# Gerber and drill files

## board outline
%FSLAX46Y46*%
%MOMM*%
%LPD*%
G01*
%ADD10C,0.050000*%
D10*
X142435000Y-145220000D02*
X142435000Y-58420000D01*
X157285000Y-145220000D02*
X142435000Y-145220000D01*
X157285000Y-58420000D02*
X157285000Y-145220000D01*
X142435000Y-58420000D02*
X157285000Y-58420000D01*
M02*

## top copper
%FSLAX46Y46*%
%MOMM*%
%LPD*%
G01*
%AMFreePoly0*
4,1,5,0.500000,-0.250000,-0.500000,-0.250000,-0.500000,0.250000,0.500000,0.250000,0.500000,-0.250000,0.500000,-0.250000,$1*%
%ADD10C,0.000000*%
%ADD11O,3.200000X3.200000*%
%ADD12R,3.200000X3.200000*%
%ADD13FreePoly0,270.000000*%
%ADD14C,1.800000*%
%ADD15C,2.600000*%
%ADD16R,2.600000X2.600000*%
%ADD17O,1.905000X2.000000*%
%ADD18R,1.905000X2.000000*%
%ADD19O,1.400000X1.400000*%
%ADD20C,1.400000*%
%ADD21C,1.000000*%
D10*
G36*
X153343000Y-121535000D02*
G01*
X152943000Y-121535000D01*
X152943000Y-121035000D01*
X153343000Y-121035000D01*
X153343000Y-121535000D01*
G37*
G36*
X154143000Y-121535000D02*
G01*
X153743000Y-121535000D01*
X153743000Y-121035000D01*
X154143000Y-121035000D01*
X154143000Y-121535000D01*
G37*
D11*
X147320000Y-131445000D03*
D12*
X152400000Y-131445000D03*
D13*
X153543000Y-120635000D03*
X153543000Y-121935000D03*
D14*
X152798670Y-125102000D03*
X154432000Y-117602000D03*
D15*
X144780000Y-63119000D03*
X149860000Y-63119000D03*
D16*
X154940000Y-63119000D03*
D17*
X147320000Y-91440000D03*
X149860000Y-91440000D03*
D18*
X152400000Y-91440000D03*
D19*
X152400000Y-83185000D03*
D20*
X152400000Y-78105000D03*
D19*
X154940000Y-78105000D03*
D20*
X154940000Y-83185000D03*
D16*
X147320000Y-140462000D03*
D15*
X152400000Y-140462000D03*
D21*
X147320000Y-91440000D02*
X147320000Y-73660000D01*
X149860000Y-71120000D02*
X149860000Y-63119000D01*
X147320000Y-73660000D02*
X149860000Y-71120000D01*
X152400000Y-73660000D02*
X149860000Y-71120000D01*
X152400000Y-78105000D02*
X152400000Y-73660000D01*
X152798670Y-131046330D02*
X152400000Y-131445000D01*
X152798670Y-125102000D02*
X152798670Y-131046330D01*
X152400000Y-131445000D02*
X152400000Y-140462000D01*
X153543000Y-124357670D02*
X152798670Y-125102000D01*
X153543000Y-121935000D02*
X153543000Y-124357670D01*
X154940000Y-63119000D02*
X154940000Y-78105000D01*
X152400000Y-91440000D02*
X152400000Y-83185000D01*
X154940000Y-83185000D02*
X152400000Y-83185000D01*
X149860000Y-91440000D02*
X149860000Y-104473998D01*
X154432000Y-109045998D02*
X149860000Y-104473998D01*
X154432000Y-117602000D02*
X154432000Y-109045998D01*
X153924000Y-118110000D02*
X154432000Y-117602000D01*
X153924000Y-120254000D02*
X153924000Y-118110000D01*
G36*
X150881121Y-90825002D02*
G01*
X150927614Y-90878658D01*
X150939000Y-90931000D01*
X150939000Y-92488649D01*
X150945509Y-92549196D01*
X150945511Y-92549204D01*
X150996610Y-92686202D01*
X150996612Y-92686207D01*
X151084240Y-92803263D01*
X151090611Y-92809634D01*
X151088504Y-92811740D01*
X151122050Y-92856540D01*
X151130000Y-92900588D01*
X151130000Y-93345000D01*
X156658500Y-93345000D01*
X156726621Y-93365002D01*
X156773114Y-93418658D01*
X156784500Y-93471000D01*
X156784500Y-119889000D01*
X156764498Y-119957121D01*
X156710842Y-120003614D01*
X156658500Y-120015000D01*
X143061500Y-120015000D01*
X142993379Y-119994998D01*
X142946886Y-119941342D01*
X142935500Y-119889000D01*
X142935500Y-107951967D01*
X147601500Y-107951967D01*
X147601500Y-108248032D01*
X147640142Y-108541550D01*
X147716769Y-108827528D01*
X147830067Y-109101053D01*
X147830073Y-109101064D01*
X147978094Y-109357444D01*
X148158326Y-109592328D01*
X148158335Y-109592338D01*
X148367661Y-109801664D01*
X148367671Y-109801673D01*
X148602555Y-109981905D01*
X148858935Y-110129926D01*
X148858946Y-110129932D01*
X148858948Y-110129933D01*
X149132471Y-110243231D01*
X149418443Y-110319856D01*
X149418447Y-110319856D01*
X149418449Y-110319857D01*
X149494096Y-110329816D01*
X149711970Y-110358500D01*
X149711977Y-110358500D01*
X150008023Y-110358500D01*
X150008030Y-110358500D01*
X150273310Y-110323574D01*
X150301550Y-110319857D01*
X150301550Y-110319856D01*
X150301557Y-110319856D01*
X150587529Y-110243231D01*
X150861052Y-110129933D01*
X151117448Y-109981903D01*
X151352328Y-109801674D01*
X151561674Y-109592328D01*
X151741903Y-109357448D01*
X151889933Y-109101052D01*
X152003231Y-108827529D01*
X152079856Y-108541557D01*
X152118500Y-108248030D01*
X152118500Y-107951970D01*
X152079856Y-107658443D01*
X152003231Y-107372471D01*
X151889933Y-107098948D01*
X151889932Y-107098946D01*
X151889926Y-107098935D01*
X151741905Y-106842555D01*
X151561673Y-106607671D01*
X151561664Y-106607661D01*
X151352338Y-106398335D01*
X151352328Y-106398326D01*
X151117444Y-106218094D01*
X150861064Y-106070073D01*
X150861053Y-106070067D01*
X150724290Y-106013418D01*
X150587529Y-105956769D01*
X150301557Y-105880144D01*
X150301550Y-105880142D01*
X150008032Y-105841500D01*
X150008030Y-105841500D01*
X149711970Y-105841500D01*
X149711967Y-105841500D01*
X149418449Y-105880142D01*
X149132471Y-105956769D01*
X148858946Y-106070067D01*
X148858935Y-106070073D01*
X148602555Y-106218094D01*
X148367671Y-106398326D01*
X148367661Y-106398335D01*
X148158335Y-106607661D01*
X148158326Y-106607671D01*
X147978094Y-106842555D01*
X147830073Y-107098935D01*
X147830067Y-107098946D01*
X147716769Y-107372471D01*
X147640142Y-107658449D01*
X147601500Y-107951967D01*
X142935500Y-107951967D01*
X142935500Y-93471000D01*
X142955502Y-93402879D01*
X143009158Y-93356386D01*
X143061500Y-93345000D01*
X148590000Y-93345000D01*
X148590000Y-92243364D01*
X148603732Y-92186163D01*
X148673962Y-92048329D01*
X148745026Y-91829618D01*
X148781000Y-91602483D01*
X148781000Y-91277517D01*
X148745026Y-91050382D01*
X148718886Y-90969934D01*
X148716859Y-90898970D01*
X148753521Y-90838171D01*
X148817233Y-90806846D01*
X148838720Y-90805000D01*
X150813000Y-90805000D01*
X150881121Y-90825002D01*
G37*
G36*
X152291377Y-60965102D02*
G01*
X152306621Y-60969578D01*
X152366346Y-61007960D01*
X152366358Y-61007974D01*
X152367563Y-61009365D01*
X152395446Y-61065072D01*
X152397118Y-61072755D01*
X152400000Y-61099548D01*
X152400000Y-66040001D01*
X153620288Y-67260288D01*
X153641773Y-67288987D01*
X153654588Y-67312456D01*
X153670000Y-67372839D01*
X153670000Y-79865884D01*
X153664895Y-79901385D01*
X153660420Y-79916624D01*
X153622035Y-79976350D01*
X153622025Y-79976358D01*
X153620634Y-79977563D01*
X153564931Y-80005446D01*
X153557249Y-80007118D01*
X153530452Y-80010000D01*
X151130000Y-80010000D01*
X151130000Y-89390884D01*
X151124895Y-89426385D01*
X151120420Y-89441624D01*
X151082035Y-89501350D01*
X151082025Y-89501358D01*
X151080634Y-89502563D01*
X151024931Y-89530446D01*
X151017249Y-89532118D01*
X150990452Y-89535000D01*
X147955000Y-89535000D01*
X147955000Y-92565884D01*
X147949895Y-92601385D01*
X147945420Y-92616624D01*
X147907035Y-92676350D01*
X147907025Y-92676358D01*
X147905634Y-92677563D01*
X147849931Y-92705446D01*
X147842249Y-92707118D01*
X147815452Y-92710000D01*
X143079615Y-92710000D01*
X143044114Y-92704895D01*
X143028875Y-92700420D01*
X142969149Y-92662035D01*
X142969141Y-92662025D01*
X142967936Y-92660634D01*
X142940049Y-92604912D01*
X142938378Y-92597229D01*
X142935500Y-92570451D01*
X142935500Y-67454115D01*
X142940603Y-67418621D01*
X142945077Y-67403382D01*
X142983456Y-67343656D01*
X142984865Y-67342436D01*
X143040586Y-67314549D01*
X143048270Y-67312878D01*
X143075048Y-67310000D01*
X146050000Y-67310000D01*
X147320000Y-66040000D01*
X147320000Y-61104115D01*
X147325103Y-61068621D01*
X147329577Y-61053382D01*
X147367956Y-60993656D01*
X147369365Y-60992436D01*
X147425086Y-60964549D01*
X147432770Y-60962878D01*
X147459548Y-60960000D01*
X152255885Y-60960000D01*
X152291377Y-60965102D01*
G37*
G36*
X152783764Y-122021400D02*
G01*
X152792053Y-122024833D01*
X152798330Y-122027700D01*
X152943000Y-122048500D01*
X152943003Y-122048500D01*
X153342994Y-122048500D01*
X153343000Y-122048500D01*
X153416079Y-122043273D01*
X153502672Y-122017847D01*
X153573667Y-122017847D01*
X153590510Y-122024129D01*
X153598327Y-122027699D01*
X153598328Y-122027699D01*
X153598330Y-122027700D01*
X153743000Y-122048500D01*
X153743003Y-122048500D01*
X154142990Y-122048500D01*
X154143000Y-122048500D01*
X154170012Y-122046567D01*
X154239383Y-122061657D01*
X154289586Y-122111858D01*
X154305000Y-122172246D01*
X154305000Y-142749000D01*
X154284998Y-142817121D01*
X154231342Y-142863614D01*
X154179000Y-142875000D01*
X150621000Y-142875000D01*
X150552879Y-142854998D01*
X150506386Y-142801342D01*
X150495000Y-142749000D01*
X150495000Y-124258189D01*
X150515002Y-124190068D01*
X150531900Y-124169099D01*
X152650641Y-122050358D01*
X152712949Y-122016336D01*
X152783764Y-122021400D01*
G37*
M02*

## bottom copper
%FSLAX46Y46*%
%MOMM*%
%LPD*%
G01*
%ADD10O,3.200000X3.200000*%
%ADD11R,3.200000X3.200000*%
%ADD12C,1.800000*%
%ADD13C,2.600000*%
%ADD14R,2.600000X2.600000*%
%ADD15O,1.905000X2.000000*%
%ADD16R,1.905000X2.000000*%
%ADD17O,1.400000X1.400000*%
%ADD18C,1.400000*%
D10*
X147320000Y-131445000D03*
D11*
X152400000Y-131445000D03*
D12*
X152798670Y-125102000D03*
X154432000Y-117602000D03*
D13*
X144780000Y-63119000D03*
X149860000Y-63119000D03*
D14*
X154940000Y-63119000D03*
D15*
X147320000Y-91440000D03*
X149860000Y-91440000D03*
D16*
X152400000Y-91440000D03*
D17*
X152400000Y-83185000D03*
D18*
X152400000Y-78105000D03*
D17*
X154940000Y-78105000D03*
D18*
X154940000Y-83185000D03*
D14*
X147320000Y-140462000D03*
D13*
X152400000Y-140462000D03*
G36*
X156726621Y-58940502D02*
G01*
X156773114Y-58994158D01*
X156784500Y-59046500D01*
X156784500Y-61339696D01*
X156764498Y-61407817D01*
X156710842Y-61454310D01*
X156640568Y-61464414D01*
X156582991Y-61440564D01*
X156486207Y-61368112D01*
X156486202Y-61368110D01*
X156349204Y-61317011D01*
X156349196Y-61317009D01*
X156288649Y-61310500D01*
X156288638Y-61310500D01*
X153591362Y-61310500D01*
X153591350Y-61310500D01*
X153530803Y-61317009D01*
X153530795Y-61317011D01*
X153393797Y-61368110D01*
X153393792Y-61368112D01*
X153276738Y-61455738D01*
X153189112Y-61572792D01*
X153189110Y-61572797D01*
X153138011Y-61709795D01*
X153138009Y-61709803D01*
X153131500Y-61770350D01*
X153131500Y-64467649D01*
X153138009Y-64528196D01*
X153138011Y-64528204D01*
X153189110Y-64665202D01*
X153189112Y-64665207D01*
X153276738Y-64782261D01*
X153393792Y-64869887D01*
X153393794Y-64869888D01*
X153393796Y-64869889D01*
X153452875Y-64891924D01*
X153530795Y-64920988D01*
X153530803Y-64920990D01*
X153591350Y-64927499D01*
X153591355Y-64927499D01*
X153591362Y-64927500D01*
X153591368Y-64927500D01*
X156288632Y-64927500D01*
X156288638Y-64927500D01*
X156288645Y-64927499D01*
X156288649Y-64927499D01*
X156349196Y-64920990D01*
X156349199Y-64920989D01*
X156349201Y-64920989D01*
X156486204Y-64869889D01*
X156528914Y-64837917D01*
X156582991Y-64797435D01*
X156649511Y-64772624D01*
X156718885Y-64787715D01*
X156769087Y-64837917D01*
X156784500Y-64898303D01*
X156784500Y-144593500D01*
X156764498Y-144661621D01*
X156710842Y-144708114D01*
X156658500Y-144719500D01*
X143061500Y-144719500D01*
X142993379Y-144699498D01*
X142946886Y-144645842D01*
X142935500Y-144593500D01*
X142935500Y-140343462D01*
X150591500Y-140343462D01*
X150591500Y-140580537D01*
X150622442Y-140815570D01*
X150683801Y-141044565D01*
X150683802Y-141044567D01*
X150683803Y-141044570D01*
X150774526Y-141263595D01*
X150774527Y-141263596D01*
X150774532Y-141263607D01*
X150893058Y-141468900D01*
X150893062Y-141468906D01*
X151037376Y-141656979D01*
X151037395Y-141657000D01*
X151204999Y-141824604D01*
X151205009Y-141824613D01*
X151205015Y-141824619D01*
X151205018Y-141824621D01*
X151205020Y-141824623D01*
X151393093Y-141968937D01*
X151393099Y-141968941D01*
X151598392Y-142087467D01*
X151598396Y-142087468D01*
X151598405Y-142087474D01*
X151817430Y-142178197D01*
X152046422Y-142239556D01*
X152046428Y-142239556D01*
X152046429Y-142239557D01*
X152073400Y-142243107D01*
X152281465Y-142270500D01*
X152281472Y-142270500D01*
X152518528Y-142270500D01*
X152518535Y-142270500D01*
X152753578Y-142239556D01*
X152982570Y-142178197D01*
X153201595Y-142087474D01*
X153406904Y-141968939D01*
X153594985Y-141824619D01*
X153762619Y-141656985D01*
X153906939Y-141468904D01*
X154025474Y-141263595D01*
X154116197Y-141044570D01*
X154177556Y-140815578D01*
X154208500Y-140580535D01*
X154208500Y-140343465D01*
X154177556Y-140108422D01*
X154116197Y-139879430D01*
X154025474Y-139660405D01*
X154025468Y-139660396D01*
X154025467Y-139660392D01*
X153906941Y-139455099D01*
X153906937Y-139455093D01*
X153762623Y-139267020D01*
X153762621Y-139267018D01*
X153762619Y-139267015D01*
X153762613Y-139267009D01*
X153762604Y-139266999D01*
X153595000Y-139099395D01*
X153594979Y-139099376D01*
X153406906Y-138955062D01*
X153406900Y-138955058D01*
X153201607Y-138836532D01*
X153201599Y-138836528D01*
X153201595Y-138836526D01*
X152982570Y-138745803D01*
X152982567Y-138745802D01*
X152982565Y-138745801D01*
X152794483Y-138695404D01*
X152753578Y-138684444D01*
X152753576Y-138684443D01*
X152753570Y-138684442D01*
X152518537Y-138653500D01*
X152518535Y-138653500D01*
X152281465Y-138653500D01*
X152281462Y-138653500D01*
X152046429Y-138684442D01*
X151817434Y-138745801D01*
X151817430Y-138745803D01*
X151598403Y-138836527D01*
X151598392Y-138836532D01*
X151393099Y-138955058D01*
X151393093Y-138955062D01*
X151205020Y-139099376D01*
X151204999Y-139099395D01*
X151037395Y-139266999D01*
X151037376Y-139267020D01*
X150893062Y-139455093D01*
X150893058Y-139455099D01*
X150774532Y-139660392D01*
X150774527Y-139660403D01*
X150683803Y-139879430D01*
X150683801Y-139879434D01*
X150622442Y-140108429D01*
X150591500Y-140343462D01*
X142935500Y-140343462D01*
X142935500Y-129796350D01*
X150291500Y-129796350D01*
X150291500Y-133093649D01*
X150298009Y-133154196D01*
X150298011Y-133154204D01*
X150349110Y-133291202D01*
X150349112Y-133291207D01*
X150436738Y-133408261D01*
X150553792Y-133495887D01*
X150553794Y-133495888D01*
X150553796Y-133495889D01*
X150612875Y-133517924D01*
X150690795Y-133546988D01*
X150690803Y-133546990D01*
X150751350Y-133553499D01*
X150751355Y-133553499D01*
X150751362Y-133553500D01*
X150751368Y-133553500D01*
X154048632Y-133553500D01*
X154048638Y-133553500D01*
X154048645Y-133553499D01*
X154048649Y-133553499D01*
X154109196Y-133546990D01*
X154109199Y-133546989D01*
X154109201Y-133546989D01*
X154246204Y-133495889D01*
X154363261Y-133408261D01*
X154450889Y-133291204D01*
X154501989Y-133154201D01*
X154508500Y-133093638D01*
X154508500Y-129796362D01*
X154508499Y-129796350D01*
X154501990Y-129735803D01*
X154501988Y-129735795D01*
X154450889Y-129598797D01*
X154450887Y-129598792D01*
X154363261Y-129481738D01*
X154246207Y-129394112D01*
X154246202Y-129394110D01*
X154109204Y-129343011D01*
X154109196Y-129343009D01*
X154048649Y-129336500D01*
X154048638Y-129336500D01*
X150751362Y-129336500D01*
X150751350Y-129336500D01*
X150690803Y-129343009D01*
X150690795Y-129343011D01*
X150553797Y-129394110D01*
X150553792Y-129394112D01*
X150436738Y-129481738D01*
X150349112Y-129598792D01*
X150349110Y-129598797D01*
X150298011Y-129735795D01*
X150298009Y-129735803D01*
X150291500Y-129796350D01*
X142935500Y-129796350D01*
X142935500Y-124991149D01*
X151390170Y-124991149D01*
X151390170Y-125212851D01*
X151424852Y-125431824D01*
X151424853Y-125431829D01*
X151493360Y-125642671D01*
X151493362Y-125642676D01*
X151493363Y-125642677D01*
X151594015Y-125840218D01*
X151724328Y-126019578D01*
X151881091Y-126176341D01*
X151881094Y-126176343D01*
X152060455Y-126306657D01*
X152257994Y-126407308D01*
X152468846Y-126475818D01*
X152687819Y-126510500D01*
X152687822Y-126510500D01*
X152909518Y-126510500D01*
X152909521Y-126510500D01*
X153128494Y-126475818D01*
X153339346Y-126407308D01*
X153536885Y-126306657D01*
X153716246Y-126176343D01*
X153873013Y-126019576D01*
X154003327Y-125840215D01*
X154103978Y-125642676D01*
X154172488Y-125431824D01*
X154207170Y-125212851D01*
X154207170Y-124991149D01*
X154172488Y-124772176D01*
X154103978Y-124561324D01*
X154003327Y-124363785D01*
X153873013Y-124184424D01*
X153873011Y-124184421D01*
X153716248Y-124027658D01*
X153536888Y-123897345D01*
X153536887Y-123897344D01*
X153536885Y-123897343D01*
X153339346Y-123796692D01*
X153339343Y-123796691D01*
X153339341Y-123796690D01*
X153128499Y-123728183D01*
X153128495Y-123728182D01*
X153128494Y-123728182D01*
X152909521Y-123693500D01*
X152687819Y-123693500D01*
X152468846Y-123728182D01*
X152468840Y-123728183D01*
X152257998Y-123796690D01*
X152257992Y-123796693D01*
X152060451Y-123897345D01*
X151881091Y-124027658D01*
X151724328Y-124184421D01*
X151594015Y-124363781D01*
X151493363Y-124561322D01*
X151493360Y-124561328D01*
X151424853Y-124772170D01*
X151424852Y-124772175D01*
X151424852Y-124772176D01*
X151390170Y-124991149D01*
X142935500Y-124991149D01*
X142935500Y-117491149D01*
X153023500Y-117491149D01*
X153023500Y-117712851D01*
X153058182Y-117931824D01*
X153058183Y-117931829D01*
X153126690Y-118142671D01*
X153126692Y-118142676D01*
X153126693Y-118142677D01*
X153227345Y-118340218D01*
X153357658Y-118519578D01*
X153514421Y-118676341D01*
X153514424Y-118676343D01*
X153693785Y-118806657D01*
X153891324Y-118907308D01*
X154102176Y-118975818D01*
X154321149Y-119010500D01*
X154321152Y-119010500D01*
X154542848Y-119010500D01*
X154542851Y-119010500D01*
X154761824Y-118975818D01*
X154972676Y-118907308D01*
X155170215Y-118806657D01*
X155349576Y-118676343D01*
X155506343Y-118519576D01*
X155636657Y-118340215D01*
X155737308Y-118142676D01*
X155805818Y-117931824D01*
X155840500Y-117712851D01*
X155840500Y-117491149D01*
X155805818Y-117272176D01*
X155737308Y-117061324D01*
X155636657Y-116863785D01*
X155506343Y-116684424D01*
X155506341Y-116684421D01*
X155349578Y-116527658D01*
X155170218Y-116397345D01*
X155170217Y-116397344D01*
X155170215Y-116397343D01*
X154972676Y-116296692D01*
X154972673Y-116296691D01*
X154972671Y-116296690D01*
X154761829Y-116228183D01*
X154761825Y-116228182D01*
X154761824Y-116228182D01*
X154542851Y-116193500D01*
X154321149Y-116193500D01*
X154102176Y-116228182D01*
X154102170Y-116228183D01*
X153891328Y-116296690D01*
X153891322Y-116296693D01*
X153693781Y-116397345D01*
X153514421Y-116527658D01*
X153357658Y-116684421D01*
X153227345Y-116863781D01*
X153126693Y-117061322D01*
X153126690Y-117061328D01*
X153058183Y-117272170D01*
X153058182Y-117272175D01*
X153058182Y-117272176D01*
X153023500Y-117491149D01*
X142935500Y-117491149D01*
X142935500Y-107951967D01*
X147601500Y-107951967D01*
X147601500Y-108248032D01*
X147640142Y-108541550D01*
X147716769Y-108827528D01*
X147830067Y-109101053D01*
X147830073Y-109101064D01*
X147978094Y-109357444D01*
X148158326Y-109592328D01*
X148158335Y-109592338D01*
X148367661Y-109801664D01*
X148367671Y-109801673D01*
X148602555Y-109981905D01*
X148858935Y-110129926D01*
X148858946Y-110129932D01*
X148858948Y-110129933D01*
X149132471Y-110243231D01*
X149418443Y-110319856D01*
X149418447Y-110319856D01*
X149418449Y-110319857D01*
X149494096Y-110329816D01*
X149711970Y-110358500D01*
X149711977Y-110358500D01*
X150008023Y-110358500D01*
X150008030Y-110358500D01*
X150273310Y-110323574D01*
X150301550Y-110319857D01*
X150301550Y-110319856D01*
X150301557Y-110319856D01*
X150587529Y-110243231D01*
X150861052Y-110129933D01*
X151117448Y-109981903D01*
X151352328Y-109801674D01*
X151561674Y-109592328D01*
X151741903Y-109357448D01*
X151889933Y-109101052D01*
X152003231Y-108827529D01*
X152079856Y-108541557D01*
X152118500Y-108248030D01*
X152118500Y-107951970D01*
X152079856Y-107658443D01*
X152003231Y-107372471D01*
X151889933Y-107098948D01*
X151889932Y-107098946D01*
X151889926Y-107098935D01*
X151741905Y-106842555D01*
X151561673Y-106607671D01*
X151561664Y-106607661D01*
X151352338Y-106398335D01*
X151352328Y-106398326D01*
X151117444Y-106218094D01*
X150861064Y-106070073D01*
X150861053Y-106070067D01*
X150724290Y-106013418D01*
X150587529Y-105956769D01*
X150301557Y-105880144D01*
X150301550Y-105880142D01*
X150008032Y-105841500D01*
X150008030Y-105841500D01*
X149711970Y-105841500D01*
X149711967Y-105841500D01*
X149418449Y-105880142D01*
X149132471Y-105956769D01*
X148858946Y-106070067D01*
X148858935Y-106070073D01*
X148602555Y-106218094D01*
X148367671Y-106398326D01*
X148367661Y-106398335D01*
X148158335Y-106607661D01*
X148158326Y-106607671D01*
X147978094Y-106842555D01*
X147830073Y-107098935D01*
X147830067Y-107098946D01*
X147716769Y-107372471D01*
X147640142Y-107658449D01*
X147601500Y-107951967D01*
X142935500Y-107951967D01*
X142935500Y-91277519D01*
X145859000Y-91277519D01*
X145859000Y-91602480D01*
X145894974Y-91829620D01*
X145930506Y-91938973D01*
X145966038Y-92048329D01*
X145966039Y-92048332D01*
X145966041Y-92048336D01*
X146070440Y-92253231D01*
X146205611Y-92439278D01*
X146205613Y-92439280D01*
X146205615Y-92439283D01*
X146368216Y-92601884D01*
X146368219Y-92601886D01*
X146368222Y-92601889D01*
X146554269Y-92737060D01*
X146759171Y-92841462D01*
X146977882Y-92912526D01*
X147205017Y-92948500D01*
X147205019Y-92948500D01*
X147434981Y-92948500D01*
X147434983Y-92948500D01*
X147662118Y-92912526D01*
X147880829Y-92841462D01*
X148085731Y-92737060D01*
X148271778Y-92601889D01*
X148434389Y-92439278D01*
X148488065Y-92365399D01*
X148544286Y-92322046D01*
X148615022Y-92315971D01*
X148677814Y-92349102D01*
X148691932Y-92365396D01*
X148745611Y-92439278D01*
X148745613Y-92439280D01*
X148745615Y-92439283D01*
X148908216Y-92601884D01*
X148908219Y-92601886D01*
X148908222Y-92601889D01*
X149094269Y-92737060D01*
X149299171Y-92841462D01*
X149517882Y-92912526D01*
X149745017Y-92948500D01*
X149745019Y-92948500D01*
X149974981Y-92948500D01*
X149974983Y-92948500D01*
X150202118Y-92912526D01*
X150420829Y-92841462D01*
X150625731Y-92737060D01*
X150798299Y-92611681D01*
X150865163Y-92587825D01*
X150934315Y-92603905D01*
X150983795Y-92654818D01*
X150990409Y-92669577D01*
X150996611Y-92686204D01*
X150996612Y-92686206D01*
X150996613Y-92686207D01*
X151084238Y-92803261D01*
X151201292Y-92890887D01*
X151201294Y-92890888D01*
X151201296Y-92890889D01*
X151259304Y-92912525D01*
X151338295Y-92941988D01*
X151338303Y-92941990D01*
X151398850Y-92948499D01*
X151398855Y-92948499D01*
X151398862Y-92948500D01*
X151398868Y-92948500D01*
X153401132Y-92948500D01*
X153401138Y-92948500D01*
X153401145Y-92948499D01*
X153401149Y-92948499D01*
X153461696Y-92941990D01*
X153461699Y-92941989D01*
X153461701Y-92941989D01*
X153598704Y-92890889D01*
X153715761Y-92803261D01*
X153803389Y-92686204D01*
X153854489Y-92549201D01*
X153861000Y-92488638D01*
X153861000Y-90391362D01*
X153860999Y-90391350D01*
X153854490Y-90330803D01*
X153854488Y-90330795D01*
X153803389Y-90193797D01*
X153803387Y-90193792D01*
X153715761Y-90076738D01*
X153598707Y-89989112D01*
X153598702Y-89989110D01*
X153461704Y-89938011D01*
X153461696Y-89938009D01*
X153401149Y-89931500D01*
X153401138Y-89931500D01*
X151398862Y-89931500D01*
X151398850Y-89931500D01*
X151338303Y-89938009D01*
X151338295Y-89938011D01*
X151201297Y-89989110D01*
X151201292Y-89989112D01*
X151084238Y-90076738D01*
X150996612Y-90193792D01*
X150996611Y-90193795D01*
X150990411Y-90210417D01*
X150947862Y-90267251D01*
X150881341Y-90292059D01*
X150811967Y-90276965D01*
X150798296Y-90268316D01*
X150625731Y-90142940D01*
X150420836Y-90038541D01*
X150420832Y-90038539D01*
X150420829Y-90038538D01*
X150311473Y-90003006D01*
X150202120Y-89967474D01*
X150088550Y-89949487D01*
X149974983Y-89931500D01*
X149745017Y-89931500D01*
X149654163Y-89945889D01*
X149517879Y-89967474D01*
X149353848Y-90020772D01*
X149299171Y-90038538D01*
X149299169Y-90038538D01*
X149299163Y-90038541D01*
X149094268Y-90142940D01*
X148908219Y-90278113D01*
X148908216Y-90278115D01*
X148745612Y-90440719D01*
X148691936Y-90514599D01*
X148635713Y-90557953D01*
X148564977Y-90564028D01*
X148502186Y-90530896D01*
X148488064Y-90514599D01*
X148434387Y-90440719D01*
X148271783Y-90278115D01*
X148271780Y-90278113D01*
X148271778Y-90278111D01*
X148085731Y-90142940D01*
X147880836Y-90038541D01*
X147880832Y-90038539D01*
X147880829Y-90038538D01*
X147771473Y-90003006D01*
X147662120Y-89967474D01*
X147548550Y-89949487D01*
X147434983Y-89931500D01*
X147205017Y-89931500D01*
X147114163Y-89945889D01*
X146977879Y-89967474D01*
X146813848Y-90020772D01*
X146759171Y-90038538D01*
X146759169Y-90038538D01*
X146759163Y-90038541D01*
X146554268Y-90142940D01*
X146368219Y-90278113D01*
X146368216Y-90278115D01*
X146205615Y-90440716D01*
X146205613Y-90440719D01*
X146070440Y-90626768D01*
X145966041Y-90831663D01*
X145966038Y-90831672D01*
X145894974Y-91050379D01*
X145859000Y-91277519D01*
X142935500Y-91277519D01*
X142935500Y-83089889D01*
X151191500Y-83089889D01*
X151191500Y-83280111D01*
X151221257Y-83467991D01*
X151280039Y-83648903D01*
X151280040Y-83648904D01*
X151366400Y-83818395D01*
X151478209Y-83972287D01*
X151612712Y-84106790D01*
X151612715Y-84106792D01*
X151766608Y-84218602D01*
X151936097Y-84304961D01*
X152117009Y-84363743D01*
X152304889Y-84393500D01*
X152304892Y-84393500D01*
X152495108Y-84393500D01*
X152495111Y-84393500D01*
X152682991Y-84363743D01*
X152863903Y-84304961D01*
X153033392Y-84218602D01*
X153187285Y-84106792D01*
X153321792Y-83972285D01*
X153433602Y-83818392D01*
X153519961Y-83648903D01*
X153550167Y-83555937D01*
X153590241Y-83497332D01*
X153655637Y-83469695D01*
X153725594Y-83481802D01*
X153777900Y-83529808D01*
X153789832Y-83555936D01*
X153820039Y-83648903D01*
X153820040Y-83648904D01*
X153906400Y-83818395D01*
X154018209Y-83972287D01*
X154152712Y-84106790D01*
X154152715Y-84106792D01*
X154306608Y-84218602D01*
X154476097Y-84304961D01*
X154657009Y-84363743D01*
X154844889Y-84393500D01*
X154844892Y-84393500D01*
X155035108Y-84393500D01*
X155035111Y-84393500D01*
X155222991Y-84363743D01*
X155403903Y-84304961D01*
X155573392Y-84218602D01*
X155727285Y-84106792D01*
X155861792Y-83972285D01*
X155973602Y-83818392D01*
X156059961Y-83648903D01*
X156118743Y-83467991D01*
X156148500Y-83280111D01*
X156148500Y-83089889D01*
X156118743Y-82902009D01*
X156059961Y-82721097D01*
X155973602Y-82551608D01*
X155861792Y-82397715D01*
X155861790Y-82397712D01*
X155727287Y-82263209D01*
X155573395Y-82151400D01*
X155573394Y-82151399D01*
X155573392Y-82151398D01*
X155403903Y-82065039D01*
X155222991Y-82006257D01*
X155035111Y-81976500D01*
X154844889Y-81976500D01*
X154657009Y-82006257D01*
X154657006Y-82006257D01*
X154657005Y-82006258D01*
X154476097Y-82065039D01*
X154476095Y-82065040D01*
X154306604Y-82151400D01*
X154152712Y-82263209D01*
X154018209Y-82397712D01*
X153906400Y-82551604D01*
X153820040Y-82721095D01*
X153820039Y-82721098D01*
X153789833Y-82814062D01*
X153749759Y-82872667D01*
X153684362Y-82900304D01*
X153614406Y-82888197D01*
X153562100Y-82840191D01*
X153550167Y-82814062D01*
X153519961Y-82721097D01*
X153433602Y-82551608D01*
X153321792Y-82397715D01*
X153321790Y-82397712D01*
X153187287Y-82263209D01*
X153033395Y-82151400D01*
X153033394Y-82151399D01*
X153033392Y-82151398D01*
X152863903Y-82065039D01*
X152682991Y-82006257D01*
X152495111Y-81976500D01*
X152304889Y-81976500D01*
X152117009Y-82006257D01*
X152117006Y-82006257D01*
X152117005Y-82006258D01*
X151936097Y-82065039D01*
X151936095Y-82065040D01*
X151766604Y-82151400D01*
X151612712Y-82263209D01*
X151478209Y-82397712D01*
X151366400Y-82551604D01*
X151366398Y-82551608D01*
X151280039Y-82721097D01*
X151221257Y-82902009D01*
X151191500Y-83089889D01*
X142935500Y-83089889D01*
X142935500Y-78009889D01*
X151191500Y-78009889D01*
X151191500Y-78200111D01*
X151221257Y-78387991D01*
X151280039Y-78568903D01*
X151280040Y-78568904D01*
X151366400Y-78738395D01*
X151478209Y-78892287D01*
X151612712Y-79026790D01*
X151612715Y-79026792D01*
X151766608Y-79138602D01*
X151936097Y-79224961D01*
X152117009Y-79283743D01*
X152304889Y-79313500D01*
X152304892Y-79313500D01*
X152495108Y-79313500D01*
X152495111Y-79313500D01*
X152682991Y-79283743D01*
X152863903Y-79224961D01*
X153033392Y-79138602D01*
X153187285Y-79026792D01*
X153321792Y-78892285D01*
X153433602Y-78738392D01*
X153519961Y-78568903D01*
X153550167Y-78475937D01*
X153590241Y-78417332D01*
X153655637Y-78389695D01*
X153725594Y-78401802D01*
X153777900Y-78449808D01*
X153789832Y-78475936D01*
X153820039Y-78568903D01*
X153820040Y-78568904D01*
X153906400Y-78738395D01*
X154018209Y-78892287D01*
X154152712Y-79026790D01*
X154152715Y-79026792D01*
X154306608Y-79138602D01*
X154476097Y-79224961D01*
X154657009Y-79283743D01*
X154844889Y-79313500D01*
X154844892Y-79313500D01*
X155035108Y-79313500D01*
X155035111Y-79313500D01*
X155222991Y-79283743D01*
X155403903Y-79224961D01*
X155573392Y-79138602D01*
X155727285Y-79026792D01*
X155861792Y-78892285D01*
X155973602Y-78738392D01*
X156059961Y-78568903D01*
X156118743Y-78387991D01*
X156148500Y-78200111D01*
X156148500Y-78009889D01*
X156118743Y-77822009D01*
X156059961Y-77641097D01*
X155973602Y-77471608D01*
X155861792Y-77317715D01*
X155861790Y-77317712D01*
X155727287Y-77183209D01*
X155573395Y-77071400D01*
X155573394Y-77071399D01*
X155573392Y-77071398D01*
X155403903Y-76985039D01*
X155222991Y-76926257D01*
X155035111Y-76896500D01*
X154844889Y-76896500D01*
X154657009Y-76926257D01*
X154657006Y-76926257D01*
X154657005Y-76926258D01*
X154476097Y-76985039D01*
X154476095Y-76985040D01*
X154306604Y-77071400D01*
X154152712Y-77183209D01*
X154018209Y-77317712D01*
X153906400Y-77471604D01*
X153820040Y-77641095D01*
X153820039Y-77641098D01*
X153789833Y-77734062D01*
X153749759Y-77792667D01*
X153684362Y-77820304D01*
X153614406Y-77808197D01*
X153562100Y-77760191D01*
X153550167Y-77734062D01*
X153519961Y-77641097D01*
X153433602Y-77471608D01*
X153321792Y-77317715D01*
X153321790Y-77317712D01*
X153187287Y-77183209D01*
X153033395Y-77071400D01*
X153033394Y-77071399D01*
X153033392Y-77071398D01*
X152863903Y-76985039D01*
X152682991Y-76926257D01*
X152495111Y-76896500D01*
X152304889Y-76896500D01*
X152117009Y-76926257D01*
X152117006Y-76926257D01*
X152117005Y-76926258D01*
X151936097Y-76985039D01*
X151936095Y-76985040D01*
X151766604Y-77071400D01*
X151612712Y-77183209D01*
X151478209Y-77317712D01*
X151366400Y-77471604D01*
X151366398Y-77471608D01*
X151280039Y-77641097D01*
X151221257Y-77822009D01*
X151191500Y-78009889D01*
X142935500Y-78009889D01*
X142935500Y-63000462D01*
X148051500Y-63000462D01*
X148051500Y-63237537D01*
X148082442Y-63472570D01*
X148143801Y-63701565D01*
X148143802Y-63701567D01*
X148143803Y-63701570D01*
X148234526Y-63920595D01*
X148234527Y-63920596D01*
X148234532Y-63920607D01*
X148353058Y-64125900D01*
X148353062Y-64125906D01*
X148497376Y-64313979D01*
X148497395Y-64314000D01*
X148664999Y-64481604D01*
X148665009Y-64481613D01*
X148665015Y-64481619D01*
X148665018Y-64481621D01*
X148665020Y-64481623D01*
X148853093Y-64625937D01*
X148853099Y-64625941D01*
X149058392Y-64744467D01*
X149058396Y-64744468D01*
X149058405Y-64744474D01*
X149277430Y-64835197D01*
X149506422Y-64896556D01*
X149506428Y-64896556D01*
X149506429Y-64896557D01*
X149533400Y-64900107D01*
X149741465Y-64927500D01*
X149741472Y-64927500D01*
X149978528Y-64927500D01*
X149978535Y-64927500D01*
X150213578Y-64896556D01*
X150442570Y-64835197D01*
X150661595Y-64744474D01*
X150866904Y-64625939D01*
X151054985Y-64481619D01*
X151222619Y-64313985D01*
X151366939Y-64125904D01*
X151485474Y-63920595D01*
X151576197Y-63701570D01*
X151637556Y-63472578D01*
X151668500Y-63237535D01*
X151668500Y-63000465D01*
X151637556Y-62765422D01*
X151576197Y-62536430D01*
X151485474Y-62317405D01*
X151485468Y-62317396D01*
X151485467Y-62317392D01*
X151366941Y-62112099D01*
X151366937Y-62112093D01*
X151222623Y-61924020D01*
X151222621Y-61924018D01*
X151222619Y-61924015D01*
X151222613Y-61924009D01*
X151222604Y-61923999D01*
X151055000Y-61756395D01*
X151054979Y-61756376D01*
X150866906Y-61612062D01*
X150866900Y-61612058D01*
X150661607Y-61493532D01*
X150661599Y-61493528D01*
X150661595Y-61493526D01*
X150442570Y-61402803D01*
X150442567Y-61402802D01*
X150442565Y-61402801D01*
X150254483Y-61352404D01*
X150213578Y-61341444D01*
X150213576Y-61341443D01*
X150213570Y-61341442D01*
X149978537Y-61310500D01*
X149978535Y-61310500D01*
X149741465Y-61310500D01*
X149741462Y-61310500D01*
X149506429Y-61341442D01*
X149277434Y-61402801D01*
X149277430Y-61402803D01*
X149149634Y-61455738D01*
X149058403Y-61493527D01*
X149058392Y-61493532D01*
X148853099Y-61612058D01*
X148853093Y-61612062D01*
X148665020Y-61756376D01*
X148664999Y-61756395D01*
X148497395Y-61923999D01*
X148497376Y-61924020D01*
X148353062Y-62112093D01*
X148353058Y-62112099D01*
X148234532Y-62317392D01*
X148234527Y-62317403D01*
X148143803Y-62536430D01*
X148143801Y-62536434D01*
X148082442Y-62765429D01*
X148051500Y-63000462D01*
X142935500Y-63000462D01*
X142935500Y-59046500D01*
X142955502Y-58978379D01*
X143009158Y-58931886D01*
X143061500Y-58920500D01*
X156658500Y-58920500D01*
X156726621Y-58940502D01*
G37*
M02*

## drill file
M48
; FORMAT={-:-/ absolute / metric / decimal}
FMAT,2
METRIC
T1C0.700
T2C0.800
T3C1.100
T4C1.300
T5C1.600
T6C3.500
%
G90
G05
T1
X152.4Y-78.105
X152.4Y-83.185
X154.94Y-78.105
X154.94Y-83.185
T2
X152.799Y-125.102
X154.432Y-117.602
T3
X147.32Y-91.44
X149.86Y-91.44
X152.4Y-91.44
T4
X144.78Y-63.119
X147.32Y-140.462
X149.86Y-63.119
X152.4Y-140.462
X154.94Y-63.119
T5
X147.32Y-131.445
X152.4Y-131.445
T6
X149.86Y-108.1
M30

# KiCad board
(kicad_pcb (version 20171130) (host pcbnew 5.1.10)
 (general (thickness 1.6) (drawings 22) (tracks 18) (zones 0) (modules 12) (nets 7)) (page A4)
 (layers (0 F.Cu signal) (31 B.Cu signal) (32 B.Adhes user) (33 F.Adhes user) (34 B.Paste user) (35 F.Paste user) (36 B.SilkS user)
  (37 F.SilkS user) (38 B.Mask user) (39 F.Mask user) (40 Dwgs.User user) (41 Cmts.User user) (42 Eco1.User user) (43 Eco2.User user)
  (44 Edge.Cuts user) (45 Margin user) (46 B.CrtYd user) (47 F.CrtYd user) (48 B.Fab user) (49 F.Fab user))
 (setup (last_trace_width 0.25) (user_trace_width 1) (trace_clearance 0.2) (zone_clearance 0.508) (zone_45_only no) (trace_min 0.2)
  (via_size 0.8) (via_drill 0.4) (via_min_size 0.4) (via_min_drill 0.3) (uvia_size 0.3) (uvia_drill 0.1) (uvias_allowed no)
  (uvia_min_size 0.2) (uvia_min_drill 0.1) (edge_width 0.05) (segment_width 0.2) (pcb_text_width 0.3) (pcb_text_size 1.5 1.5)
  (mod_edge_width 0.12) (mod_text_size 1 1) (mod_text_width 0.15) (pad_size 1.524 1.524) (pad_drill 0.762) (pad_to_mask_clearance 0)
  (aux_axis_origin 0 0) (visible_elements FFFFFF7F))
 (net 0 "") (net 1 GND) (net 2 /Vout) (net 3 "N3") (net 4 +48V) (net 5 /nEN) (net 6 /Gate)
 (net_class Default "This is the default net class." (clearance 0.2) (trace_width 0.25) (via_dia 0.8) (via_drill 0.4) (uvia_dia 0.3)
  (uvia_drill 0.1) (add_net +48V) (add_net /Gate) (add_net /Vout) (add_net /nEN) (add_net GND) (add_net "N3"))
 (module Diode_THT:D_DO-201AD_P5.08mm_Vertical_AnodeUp (layer F.Cu) (at 152.4 131.445 180)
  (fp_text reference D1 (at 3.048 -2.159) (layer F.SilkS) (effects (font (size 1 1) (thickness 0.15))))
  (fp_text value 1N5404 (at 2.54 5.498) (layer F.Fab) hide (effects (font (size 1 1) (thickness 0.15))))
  (pad 2 thru_hole oval (at 5.08 0 180) (size 3.2 3.2) (drill 1.6) (layers *.Cu *.Mask) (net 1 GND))
  (pad 1 thru_hole rect (at 0 0 180) (size 3.2 3.2) (drill 1.6) (layers *.Cu *.Mask) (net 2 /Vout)))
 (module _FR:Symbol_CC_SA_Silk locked (layer B.Cu) (at 146.304 86.487 180)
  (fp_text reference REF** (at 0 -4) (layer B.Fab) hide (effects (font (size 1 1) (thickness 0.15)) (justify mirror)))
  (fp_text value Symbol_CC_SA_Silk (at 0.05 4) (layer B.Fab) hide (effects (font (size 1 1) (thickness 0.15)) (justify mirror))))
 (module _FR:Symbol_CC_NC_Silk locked (layer B.Cu) (at 146.304 79.375 180)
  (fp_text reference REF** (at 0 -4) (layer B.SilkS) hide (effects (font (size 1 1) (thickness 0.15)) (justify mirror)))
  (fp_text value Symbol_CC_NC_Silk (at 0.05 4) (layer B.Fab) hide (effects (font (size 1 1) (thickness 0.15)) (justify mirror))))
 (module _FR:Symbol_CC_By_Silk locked (layer B.Cu) (at 146.304 72.39 180)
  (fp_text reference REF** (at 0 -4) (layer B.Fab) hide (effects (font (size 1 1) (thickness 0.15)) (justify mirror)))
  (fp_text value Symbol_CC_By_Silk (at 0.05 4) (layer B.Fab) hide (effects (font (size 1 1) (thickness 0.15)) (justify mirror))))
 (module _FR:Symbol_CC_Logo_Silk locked (layer B.Cu) (at 153.289 72.263 180)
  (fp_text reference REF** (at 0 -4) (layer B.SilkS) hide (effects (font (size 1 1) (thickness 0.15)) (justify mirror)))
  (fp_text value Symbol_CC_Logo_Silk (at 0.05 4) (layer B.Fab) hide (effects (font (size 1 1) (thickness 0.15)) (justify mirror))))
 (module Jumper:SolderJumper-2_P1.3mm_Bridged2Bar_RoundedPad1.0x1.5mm (layer F.Cu) (at 153.543 121.285 270)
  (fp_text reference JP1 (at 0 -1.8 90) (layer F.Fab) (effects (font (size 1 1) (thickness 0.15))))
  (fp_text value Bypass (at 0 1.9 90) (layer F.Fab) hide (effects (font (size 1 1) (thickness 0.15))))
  (fp_poly (pts (xy -0.25 0.2) (xy 0.25 0.2) (xy 0.25 0.6) (xy -0.25 0.6)) (layer F.Cu) (width 0))
  (fp_poly (pts (xy -0.25 -0.6) (xy 0.25 -0.6) (xy 0.25 -0.2) (xy -0.25 -0.2)) (layer F.Cu) (width 0))
  (pad 1 smd custom (at -0.65 0 270) (size 1 0.5) (layers F.Cu F.Mask) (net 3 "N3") (zone_connect 2)
   (options (clearance outline) (anchor rect)) (primitives))
  (pad 2 smd custom (at 0.65 0 270) (size 1 0.5) (layers F.Cu F.Mask) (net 2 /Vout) (zone_connect 2)
   (options (clearance outline) (anchor rect)) (primitives)))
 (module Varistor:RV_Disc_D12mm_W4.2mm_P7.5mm (layer F.Cu) (at 154.432 117.602 270)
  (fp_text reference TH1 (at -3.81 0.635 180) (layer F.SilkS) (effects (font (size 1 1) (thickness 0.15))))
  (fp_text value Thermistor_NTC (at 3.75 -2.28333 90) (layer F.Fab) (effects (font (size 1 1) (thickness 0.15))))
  (pad 2 thru_hole circle (at 7.5 1.63333 270) (size 1.8 1.8) (drill 0.8) (layers *.Cu *.Mask) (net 2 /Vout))
  (pad 1 thru_hole circle (at 0 0 270) (size 1.8 1.8) (drill 0.8) (layers *.Cu *.Mask) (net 3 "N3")))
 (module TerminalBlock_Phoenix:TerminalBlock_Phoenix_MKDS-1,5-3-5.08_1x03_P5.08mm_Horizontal (layer F.Cu) (at 154.94 63.119 180)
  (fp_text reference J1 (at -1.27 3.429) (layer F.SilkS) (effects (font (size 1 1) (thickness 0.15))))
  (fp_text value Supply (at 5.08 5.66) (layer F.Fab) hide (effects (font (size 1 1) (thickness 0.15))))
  (pad 3 thru_hole circle (at 10.16 0 180) (size 2.6 2.6) (drill 1.3) (layers *.Cu *.Mask) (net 1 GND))
  (pad 2 thru_hole circle (at 5.08 0 180) (size 2.6 2.6) (drill 1.3) (layers *.Cu *.Mask) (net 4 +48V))
  (pad 1 thru_hole rect (at 0 0 180) (size 2.6 2.6) (drill 1.3) (layers *.Cu *.Mask) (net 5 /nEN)))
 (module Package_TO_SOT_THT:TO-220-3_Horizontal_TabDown (layer F.Cu) (at 152.4 91.44 180)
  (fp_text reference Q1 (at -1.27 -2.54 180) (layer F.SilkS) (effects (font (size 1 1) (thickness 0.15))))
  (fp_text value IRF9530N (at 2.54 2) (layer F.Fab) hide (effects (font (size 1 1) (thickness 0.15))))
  (pad 3 thru_hole oval (at 5.08 0 180) (size 1.905 2) (drill 1.1) (layers *.Cu *.Mask) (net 4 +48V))
  (pad 2 thru_hole oval (at 2.54 0 180) (size 1.905 2) (drill 1.1) (layers *.Cu *.Mask) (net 3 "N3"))
  (pad 1 thru_hole rect (at 0 0 180) (size 1.905 2) (drill 1.1) (layers *.Cu *.Mask) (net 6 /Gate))
  (pad "" np_thru_hole oval (at 2.54 -16.66 180) (size 3.5 3.5) (drill 3.5) (layers *.Cu *.Mask)))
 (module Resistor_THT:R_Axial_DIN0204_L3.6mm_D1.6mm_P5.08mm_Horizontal (layer F.Cu) (at 152.4 78.105 270)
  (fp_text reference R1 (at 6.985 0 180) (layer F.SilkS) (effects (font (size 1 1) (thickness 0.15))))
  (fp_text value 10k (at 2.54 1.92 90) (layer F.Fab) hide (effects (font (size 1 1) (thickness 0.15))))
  (pad 2 thru_hole oval (at 5.08 0 270) (size 1.4 1.4) (drill 0.7) (layers *.Cu *.Mask) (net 6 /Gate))
  (pad 1 thru_hole circle (at 0 0 270) (size 1.4 1.4) (drill 0.7) (layers *.Cu *.Mask) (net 4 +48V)))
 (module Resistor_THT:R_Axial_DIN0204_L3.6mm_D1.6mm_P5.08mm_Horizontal (layer F.Cu) (at 154.94 83.185 90)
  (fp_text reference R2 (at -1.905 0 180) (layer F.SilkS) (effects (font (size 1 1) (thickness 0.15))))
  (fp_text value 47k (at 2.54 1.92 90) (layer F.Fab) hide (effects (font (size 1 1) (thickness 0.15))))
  (pad 2 thru_hole oval (at 5.08 0 90) (size 1.4 1.4) (drill 0.7) (layers *.Cu *.Mask) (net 5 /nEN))
  (pad 1 thru_hole circle (at 0 0 90) (size 1.4 1.4) (drill 0.7) (layers *.Cu *.Mask) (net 6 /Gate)))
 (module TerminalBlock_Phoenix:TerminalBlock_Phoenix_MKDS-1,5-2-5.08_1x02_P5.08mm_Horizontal (layer F.Cu) (at 147.32 140.462)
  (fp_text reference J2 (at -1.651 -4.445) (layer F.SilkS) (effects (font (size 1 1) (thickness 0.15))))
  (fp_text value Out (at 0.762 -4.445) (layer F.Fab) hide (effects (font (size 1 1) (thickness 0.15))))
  (pad 1 thru_hole rect (at 0 0) (size 2.6 2.6) (drill 1.3) (layers *.Cu *.Mask) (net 1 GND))
  (pad 2 thru_hole circle (at 5.08 0) (size 2.6 2.6) (drill 1.3) (layers *.Cu *.Mask) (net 2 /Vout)))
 (gr_line (start 142.435 145.22) (end 142.435 58.42) (layer Edge.Cuts) (width 0.05))
 (gr_line (start 157.285 145.22) (end 142.435 145.22) (layer Edge.Cuts) (width 0.05))
 (gr_line (start 157.285 58.42) (end 157.285 145.22) (layer Edge.Cuts) (width 0.05))
 (gr_line (start 142.435 58.42) (end 157.285 58.42) (layer Edge.Cuts) (width 0.05))
 (segment (start 147.32 91.44) (end 147.32 73.66) (width 1) (layer F.Cu) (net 4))
 (segment (start 149.86 71.12) (end 149.86 63.119) (width 1) (layer F.Cu) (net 4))
 (segment (start 147.32 73.66) (end 149.86 71.12) (width 1) (layer F.Cu) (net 4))
 (segment (start 152.4 73.66) (end 149.86 71.12) (width 1) (layer F.Cu) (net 4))
 (segment (start 152.4 78.105) (end 152.4 73.66) (width 1) (layer F.Cu) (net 4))
 (segment (start 152.79867 131.04633) (end 152.4 131.445) (width 1) (layer F.Cu) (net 2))
 (segment (start 152.79867 125.102) (end 152.79867 131.04633) (width 1) (layer F.Cu) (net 2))
 (segment (start 152.4 131.445) (end 152.4 140.462) (width 1) (layer F.Cu) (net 2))
 (segment (start 153.543 124.35767) (end 152.79867 125.102) (width 1) (layer F.Cu) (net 2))
 (segment (start 153.543 121.935) (end 153.543 124.35767) (width 1) (layer F.Cu) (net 2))
 (segment (start 154.94 63.119) (end 154.94 78.105) (width 1) (layer F.Cu) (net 5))
 (segment (start 152.4 91.44) (end 152.4 83.185) (width 1) (layer F.Cu) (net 6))
 (segment (start 154.94 83.185) (end 152.4 83.185) (width 1) (layer F.Cu) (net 6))
 (segment (start 149.86 91.44) (end 149.86 104.473998) (width 1) (layer F.Cu) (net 3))
 (segment (start 154.432 109.045998) (end 149.86 104.473998) (width 1) (layer F.Cu) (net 3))
 (segment (start 154.432 117.602) (end 154.432 109.045998) (width 1) (layer F.Cu) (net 3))
 (segment (start 153.924 118.11) (end 154.432 117.602) (width 1) (layer F.Cu) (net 3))
 (segment (start 153.924 120.254) (end 153.924 118.11) (width 1) (layer F.Cu) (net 3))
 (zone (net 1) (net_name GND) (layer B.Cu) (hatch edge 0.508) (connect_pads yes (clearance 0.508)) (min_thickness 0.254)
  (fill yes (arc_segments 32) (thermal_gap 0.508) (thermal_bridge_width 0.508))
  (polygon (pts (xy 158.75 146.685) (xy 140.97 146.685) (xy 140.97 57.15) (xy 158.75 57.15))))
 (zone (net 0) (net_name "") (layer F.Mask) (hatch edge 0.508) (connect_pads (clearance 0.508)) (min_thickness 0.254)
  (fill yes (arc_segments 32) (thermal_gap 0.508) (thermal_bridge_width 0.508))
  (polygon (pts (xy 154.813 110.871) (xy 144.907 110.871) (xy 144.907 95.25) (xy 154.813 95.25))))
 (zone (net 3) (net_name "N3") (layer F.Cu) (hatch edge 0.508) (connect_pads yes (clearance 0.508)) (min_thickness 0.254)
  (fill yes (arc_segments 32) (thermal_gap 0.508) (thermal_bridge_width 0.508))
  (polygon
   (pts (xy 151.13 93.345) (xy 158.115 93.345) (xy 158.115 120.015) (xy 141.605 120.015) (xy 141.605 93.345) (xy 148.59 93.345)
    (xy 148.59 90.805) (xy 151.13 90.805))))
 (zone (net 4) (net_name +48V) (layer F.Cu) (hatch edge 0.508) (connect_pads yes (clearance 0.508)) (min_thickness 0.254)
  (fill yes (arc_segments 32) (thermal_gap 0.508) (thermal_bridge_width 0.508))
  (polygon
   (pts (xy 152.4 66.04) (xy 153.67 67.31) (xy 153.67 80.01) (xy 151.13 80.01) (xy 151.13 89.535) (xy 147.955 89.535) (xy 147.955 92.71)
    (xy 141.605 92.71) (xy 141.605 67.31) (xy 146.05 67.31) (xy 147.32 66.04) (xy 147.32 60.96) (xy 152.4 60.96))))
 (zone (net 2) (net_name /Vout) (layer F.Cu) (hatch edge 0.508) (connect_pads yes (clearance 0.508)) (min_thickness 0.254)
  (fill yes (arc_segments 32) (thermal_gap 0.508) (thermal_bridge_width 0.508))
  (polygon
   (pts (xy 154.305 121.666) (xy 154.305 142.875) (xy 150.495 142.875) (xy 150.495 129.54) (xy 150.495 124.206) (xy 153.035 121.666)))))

